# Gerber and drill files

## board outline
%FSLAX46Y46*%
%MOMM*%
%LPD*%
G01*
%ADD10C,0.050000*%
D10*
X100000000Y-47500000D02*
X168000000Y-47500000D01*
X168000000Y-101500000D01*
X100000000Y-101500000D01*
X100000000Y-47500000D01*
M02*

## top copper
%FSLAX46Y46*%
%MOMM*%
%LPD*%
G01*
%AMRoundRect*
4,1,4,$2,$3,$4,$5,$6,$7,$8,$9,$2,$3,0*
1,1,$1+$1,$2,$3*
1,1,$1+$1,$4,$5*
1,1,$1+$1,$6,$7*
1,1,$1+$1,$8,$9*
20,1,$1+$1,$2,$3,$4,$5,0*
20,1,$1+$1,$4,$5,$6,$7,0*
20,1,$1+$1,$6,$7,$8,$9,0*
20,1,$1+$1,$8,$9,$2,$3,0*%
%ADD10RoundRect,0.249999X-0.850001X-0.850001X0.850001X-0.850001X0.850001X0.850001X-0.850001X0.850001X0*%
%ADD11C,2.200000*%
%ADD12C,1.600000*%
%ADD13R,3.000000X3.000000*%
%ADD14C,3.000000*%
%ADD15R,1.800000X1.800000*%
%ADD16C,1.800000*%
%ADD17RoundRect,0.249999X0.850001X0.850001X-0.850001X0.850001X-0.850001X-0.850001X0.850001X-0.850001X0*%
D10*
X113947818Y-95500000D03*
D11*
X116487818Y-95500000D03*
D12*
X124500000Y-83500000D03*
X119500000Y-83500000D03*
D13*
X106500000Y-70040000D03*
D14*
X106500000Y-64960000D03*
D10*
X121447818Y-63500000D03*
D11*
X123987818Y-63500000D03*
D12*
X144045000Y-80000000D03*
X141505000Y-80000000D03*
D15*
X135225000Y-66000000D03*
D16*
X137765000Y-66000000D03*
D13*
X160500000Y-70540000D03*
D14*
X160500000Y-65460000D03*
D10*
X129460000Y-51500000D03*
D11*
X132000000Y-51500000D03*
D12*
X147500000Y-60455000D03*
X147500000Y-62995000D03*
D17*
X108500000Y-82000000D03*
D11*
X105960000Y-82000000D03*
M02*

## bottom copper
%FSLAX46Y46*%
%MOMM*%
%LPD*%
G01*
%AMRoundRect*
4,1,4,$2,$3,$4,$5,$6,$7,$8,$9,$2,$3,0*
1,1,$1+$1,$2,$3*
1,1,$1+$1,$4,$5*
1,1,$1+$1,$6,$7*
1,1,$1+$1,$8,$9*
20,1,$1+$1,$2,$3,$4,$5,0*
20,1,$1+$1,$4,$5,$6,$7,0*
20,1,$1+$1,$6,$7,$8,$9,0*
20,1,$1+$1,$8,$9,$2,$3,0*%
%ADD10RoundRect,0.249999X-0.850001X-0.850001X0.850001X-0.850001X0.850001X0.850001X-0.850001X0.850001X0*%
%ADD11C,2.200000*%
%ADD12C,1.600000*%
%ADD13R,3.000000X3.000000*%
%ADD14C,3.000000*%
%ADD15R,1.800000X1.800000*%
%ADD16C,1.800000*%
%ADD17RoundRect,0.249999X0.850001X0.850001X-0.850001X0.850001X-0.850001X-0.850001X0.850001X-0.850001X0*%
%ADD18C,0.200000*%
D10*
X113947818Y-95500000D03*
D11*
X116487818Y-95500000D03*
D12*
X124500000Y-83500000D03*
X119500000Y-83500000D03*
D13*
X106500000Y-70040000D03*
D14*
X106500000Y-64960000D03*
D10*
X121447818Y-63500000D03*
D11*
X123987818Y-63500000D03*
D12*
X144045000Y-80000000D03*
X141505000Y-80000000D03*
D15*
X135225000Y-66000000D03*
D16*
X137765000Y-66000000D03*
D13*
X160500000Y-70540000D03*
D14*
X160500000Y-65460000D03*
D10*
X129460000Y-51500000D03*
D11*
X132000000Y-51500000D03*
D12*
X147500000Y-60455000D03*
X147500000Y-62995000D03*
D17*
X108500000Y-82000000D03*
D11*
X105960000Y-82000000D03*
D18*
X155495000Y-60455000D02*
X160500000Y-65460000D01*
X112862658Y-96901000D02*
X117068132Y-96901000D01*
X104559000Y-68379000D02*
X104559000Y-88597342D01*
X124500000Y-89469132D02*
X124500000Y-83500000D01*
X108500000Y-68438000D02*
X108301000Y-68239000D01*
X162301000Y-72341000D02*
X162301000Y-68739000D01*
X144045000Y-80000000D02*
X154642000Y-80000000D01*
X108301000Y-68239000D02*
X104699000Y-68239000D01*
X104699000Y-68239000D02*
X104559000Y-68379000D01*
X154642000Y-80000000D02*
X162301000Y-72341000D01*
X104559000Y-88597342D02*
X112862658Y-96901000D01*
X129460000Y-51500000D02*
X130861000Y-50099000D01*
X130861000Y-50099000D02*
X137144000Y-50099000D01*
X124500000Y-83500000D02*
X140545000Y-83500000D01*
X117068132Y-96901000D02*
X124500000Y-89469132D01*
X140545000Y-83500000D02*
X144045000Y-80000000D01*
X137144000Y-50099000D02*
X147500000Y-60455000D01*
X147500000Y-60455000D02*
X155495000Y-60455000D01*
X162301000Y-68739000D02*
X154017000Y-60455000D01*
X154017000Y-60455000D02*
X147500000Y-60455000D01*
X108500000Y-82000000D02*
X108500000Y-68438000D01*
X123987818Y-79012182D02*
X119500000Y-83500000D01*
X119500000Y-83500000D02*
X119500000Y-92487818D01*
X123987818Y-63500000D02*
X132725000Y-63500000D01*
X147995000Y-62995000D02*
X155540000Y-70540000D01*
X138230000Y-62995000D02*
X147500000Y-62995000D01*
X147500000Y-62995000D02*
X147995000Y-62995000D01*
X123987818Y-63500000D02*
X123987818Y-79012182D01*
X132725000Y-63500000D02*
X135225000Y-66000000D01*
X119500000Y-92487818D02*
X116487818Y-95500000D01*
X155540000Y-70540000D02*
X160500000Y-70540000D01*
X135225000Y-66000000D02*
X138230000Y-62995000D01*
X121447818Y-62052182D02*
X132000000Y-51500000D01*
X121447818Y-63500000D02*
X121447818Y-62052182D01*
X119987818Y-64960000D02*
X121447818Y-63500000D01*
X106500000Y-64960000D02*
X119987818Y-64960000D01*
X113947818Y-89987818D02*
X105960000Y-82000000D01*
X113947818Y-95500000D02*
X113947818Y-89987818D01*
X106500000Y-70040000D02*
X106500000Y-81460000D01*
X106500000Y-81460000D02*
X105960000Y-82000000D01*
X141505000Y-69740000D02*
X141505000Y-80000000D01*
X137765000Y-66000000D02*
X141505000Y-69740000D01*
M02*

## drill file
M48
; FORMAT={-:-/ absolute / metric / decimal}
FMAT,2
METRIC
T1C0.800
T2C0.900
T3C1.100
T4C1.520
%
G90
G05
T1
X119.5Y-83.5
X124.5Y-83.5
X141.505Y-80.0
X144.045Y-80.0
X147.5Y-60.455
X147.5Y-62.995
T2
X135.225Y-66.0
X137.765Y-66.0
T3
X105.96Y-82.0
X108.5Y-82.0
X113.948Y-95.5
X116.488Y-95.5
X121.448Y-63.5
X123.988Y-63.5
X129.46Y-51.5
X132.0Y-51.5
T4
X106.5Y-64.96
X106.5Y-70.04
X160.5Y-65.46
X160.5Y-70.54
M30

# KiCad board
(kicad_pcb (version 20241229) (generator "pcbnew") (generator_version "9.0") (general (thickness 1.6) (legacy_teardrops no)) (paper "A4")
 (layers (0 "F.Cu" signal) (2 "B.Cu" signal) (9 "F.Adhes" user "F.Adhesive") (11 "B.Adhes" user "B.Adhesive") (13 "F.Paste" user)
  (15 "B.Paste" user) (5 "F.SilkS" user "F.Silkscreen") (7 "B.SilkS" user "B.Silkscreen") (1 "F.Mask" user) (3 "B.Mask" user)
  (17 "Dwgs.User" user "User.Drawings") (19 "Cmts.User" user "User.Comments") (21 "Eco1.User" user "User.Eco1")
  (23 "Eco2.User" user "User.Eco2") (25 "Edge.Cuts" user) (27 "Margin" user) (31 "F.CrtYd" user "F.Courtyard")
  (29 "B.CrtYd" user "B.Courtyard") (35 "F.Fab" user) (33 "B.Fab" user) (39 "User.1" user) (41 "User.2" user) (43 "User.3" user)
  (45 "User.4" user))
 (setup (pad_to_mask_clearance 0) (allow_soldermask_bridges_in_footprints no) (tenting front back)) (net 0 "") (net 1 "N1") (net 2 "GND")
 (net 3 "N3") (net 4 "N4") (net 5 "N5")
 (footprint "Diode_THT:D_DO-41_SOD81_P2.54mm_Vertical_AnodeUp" (layer "F.Cu") (at 113.947818 95.5)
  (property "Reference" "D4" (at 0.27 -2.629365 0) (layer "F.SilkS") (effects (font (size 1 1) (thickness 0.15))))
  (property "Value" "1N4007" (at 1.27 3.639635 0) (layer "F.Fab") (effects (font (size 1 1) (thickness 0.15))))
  (pad "1" thru_hole roundrect (at 0 0) (size 2.2 2.2) (drill 1.1) (layers "*.Cu" "*.Mask") (remove_unused_layers no)
   (roundrect_rratio 0.113636) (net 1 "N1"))
  (pad "2" thru_hole circle (at 2.54 0) (size 2.2 2.2) (drill 1.1) (layers "*.Cu" "*.Mask") (remove_unused_layers no) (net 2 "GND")))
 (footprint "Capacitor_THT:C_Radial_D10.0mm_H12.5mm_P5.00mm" (layer "F.Cu") (at 124.5 83.5 180)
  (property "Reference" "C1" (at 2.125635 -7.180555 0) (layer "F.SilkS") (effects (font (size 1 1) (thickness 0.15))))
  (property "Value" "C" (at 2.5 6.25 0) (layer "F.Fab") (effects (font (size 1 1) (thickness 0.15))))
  (pad "1" thru_hole circle (at 0 0 180) (size 1.6 1.6) (drill 0.8) (layers "*.Cu" "*.Mask") (remove_unused_layers no) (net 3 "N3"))
  (pad "2" thru_hole circle (at 5 0 180) (size 1.6 1.6) (drill 0.8) (layers "*.Cu" "*.Mask") (remove_unused_layers no) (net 2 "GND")))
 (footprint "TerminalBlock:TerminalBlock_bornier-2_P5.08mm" (layer "F.Cu") (at 106.5 70.04 90)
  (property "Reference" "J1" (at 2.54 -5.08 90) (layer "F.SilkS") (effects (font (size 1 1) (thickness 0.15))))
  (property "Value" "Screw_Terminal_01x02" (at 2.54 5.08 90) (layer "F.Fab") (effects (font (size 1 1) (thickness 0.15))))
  (pad "1" thru_hole rect (at 0 0 90) (size 3 3) (drill 1.52) (layers "*.Cu" "*.Mask") (remove_unused_layers no) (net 1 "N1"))
  (pad "2" thru_hole circle (at 5.08 0 90) (size 3 3) (drill 1.52) (layers "*.Cu" "*.Mask") (remove_unused_layers no) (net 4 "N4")))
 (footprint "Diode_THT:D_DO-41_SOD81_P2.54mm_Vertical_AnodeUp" (layer "F.Cu") (at 121.447818 63.5)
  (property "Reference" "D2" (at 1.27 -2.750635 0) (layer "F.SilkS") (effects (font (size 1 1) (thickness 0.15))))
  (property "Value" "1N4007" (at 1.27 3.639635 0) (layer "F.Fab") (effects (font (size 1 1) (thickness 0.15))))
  (pad "1" thru_hole roundrect (at 0 0) (size 2.2 2.2) (drill 1.1) (layers "*.Cu" "*.Mask") (remove_unused_layers no)
   (roundrect_rratio 0.113636) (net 4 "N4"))
  (pad "2" thru_hole circle (at 2.54 0) (size 2.2 2.2) (drill 1.1) (layers "*.Cu" "*.Mask") (remove_unused_layers no) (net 2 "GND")))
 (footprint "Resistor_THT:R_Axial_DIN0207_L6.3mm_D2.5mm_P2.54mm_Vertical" (layer "F.Cu") (at 144.045 80 180)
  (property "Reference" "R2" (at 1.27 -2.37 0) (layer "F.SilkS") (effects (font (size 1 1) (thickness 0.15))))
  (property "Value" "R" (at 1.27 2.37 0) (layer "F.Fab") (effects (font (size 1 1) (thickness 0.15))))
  (pad "1" thru_hole circle (at 0 0 180) (size 1.6 1.6) (drill 0.8) (layers "*.Cu" "*.Mask") (remove_unused_layers no) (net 3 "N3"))
  (pad "2" thru_hole circle (at 2.54 0 180) (size 1.6 1.6) (drill 0.8) (layers "*.Cu" "*.Mask") (remove_unused_layers no) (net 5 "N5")))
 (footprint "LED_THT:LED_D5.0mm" (layer "F.Cu") (at 135.225 66)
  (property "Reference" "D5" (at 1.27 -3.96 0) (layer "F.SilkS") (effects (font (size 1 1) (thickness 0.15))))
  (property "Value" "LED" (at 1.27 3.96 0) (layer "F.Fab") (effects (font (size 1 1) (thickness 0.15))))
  (pad "1" thru_hole rect (at 0 0) (size 1.8 1.8) (drill 0.9) (layers "*.Cu" "*.Mask") (remove_unused_layers no) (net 2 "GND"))
  (pad "2" thru_hole circle (at 2.54 0) (size 1.8 1.8) (drill 0.9) (layers "*.Cu" "*.Mask") (remove_unused_layers no) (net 5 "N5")))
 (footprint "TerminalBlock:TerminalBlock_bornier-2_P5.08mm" (layer "F.Cu") (at 160.5 70.54 90)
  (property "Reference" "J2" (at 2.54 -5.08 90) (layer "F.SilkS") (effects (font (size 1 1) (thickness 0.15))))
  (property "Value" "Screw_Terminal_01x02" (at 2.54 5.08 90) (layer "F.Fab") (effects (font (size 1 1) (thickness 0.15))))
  (pad "1" thru_hole rect (at 0 0 90) (size 3 3) (drill 1.52) (layers "*.Cu" "*.Mask") (remove_unused_layers no) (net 2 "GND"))
  (pad "2" thru_hole circle (at 5.08 0 90) (size 3 3) (drill 1.52) (layers "*.Cu" "*.Mask") (remove_unused_layers no) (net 3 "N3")))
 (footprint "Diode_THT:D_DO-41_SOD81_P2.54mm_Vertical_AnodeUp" (layer "F.Cu") (at 129.46 51.5)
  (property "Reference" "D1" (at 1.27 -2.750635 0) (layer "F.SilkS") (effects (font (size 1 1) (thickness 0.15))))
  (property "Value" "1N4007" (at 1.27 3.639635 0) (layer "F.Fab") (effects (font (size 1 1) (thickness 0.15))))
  (pad "1" thru_hole roundrect (at 0 0) (size 2.2 2.2) (drill 1.1) (layers "*.Cu" "*.Mask") (remove_unused_layers no)
   (roundrect_rratio 0.113636) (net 3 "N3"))
  (pad "2" thru_hole circle (at 2.54 0) (size 2.2 2.2) (drill 1.1) (layers "*.Cu" "*.Mask") (remove_unused_layers no) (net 4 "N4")))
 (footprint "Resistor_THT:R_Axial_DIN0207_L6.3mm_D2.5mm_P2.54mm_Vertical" (layer "F.Cu") (at 147.5 60.455 -90)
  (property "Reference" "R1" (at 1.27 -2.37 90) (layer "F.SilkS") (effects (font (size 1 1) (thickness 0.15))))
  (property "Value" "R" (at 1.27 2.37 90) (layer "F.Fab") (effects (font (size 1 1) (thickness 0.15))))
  (pad "1" thru_hole circle (at 0 0 270) (size 1.6 1.6) (drill 0.8) (layers "*.Cu" "*.Mask") (remove_unused_layers no) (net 3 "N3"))
  (pad "2" thru_hole circle (at 2.54 0 270) (size 1.6 1.6) (drill 0.8) (layers "*.Cu" "*.Mask") (remove_unused_layers no) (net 2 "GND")))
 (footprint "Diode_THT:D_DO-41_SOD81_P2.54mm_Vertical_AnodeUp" (layer "F.Cu") (at 108.5 82 180)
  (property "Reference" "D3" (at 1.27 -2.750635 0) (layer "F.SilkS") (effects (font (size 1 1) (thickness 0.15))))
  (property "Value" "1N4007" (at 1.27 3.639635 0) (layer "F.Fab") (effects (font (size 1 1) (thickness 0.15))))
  (pad "1" thru_hole roundrect (at 0 0 180) (size 2.2 2.2) (drill 1.1) (layers "*.Cu" "*.Mask") (remove_unused_layers no)
   (roundrect_rratio 0.113636) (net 3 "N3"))
  (pad "2" thru_hole circle (at 2.54 0 180) (size 2.2 2.2) (drill 1.1) (layers "*.Cu" "*.Mask") (remove_unused_layers no) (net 1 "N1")))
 (gr_rect (start 100 47.5) (end 168 101.5) (stroke (width 0.05) (type default)) (fill no) (layer "Edge.Cuts"))
 (segment (start 155.495 60.455) (end 160.5 65.46) (width 0.2) (layer "B.Cu") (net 3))
 (segment (start 112.862658 96.901) (end 117.068132 96.901) (width 0.2) (layer "B.Cu") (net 3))
 (segment (start 104.559 68.379) (end 104.559 88.597342) (width 0.2) (layer "B.Cu") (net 3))
 (segment (start 124.5 89.469132) (end 124.5 83.5) (width 0.2) (layer "B.Cu") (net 3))
 (segment (start 108.5 68.438) (end 108.301 68.239) (width 0.2) (layer "B.Cu") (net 3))
 (segment (start 162.301 72.341) (end 162.301 68.739) (width 0.2) (layer "B.Cu") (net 3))
 (segment (start 144.045 80) (end 154.642 80) (width 0.2) (layer "B.Cu") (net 3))
 (segment (start 108.301 68.239) (end 104.699 68.239) (width 0.2) (layer "B.Cu") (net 3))
 (segment (start 104.699 68.239) (end 104.559 68.379) (width 0.2) (layer "B.Cu") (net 3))
 (segment (start 154.642 80) (end 162.301 72.341) (width 0.2) (layer "B.Cu") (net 3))
 (segment (start 104.559 88.597342) (end 112.862658 96.901) (width 0.2) (layer "B.Cu") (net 3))
 (segment (start 129.46 51.5) (end 130.861 50.099) (width 0.2) (layer "B.Cu") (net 3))
 (segment (start 130.861 50.099) (end 137.144 50.099) (width 0.2) (layer "B.Cu") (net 3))
 (segment (start 124.5 83.5) (end 140.545 83.5) (width 0.2) (layer "B.Cu") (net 3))
 (segment (start 117.068132 96.901) (end 124.5 89.469132) (width 0.2) (layer "B.Cu") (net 3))
 (segment (start 140.545 83.5) (end 144.045 80) (width 0.2) (layer "B.Cu") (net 3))
 (segment (start 137.144 50.099) (end 147.5 60.455) (width 0.2) (layer "B.Cu") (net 3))
 (segment (start 147.5 60.455) (end 155.495 60.455) (width 0.2) (layer "B.Cu") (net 3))
 (segment (start 162.301 68.739) (end 154.017 60.455) (width 0.2) (layer "B.Cu") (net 3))
 (segment (start 154.017 60.455) (end 147.5 60.455) (width 0.2) (layer "B.Cu") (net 3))
 (segment (start 108.5 82) (end 108.5 68.438) (width 0.2) (layer "B.Cu") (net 3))
 (segment (start 123.987818 79.012182) (end 119.5 83.5) (width 0.2) (layer "B.Cu") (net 2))
 (segment (start 119.5 83.5) (end 119.5 92.487818) (width 0.2) (layer "B.Cu") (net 2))
 (segment (start 123.987818 63.5) (end 132.725 63.5) (width 0.2) (layer "B.Cu") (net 2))
 (segment (start 147.995 62.995) (end 155.54 70.54) (width 0.2) (layer "B.Cu") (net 2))
 (segment (start 138.23 62.995) (end 147.5 62.995) (width 0.2) (layer "B.Cu") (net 2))
 (segment (start 147.5 62.995) (end 147.995 62.995) (width 0.2) (layer "B.Cu") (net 2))
 (segment (start 123.987818 63.5) (end 123.987818 79.012182) (width 0.2) (layer "B.Cu") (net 2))
 (segment (start 132.725 63.5) (end 135.225 66) (width 0.2) (layer "B.Cu") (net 2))
 (segment (start 119.5 92.487818) (end 116.487818 95.5) (width 0.2) (layer "B.Cu") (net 2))
 (segment (start 155.54 70.54) (end 160.5 70.54) (width 0.2) (layer "B.Cu") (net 2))
 (segment (start 135.225 66) (end 138.23 62.995) (width 0.2) (layer "B.Cu") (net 2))
 (segment (start 121.447818 62.052182) (end 132 51.5) (width 0.2) (layer "B.Cu") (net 4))
 (segment (start 121.447818 63.5) (end 121.447818 62.052182) (width 0.2) (layer "B.Cu") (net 4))
 (segment (start 119.987818 64.96) (end 121.447818 63.5) (width 0.2) (layer "B.Cu") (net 4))
 (segment (start 106.5 64.96) (end 119.987818 64.96) (width 0.2) (layer "B.Cu") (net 4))
 (segment (start 113.947818 89.987818) (end 105.96 82) (width 0.2) (layer "B.Cu") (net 1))
 (segment (start 113.947818 95.5) (end 113.947818 89.987818) (width 0.2) (layer "B.Cu") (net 1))
 (segment (start 106.5 70.04) (end 106.5 81.46) (width 0.2) (layer "B.Cu") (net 1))
 (segment (start 106.5 81.46) (end 105.96 82) (width 0.2) (layer "B.Cu") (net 1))
 (segment (start 141.505 69.74) (end 141.505 80) (width 0.2) (layer "B.Cu") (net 5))
 (segment (start 137.765 66) (end 141.505 69.74) (width 0.2) (layer "B.Cu") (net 5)))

